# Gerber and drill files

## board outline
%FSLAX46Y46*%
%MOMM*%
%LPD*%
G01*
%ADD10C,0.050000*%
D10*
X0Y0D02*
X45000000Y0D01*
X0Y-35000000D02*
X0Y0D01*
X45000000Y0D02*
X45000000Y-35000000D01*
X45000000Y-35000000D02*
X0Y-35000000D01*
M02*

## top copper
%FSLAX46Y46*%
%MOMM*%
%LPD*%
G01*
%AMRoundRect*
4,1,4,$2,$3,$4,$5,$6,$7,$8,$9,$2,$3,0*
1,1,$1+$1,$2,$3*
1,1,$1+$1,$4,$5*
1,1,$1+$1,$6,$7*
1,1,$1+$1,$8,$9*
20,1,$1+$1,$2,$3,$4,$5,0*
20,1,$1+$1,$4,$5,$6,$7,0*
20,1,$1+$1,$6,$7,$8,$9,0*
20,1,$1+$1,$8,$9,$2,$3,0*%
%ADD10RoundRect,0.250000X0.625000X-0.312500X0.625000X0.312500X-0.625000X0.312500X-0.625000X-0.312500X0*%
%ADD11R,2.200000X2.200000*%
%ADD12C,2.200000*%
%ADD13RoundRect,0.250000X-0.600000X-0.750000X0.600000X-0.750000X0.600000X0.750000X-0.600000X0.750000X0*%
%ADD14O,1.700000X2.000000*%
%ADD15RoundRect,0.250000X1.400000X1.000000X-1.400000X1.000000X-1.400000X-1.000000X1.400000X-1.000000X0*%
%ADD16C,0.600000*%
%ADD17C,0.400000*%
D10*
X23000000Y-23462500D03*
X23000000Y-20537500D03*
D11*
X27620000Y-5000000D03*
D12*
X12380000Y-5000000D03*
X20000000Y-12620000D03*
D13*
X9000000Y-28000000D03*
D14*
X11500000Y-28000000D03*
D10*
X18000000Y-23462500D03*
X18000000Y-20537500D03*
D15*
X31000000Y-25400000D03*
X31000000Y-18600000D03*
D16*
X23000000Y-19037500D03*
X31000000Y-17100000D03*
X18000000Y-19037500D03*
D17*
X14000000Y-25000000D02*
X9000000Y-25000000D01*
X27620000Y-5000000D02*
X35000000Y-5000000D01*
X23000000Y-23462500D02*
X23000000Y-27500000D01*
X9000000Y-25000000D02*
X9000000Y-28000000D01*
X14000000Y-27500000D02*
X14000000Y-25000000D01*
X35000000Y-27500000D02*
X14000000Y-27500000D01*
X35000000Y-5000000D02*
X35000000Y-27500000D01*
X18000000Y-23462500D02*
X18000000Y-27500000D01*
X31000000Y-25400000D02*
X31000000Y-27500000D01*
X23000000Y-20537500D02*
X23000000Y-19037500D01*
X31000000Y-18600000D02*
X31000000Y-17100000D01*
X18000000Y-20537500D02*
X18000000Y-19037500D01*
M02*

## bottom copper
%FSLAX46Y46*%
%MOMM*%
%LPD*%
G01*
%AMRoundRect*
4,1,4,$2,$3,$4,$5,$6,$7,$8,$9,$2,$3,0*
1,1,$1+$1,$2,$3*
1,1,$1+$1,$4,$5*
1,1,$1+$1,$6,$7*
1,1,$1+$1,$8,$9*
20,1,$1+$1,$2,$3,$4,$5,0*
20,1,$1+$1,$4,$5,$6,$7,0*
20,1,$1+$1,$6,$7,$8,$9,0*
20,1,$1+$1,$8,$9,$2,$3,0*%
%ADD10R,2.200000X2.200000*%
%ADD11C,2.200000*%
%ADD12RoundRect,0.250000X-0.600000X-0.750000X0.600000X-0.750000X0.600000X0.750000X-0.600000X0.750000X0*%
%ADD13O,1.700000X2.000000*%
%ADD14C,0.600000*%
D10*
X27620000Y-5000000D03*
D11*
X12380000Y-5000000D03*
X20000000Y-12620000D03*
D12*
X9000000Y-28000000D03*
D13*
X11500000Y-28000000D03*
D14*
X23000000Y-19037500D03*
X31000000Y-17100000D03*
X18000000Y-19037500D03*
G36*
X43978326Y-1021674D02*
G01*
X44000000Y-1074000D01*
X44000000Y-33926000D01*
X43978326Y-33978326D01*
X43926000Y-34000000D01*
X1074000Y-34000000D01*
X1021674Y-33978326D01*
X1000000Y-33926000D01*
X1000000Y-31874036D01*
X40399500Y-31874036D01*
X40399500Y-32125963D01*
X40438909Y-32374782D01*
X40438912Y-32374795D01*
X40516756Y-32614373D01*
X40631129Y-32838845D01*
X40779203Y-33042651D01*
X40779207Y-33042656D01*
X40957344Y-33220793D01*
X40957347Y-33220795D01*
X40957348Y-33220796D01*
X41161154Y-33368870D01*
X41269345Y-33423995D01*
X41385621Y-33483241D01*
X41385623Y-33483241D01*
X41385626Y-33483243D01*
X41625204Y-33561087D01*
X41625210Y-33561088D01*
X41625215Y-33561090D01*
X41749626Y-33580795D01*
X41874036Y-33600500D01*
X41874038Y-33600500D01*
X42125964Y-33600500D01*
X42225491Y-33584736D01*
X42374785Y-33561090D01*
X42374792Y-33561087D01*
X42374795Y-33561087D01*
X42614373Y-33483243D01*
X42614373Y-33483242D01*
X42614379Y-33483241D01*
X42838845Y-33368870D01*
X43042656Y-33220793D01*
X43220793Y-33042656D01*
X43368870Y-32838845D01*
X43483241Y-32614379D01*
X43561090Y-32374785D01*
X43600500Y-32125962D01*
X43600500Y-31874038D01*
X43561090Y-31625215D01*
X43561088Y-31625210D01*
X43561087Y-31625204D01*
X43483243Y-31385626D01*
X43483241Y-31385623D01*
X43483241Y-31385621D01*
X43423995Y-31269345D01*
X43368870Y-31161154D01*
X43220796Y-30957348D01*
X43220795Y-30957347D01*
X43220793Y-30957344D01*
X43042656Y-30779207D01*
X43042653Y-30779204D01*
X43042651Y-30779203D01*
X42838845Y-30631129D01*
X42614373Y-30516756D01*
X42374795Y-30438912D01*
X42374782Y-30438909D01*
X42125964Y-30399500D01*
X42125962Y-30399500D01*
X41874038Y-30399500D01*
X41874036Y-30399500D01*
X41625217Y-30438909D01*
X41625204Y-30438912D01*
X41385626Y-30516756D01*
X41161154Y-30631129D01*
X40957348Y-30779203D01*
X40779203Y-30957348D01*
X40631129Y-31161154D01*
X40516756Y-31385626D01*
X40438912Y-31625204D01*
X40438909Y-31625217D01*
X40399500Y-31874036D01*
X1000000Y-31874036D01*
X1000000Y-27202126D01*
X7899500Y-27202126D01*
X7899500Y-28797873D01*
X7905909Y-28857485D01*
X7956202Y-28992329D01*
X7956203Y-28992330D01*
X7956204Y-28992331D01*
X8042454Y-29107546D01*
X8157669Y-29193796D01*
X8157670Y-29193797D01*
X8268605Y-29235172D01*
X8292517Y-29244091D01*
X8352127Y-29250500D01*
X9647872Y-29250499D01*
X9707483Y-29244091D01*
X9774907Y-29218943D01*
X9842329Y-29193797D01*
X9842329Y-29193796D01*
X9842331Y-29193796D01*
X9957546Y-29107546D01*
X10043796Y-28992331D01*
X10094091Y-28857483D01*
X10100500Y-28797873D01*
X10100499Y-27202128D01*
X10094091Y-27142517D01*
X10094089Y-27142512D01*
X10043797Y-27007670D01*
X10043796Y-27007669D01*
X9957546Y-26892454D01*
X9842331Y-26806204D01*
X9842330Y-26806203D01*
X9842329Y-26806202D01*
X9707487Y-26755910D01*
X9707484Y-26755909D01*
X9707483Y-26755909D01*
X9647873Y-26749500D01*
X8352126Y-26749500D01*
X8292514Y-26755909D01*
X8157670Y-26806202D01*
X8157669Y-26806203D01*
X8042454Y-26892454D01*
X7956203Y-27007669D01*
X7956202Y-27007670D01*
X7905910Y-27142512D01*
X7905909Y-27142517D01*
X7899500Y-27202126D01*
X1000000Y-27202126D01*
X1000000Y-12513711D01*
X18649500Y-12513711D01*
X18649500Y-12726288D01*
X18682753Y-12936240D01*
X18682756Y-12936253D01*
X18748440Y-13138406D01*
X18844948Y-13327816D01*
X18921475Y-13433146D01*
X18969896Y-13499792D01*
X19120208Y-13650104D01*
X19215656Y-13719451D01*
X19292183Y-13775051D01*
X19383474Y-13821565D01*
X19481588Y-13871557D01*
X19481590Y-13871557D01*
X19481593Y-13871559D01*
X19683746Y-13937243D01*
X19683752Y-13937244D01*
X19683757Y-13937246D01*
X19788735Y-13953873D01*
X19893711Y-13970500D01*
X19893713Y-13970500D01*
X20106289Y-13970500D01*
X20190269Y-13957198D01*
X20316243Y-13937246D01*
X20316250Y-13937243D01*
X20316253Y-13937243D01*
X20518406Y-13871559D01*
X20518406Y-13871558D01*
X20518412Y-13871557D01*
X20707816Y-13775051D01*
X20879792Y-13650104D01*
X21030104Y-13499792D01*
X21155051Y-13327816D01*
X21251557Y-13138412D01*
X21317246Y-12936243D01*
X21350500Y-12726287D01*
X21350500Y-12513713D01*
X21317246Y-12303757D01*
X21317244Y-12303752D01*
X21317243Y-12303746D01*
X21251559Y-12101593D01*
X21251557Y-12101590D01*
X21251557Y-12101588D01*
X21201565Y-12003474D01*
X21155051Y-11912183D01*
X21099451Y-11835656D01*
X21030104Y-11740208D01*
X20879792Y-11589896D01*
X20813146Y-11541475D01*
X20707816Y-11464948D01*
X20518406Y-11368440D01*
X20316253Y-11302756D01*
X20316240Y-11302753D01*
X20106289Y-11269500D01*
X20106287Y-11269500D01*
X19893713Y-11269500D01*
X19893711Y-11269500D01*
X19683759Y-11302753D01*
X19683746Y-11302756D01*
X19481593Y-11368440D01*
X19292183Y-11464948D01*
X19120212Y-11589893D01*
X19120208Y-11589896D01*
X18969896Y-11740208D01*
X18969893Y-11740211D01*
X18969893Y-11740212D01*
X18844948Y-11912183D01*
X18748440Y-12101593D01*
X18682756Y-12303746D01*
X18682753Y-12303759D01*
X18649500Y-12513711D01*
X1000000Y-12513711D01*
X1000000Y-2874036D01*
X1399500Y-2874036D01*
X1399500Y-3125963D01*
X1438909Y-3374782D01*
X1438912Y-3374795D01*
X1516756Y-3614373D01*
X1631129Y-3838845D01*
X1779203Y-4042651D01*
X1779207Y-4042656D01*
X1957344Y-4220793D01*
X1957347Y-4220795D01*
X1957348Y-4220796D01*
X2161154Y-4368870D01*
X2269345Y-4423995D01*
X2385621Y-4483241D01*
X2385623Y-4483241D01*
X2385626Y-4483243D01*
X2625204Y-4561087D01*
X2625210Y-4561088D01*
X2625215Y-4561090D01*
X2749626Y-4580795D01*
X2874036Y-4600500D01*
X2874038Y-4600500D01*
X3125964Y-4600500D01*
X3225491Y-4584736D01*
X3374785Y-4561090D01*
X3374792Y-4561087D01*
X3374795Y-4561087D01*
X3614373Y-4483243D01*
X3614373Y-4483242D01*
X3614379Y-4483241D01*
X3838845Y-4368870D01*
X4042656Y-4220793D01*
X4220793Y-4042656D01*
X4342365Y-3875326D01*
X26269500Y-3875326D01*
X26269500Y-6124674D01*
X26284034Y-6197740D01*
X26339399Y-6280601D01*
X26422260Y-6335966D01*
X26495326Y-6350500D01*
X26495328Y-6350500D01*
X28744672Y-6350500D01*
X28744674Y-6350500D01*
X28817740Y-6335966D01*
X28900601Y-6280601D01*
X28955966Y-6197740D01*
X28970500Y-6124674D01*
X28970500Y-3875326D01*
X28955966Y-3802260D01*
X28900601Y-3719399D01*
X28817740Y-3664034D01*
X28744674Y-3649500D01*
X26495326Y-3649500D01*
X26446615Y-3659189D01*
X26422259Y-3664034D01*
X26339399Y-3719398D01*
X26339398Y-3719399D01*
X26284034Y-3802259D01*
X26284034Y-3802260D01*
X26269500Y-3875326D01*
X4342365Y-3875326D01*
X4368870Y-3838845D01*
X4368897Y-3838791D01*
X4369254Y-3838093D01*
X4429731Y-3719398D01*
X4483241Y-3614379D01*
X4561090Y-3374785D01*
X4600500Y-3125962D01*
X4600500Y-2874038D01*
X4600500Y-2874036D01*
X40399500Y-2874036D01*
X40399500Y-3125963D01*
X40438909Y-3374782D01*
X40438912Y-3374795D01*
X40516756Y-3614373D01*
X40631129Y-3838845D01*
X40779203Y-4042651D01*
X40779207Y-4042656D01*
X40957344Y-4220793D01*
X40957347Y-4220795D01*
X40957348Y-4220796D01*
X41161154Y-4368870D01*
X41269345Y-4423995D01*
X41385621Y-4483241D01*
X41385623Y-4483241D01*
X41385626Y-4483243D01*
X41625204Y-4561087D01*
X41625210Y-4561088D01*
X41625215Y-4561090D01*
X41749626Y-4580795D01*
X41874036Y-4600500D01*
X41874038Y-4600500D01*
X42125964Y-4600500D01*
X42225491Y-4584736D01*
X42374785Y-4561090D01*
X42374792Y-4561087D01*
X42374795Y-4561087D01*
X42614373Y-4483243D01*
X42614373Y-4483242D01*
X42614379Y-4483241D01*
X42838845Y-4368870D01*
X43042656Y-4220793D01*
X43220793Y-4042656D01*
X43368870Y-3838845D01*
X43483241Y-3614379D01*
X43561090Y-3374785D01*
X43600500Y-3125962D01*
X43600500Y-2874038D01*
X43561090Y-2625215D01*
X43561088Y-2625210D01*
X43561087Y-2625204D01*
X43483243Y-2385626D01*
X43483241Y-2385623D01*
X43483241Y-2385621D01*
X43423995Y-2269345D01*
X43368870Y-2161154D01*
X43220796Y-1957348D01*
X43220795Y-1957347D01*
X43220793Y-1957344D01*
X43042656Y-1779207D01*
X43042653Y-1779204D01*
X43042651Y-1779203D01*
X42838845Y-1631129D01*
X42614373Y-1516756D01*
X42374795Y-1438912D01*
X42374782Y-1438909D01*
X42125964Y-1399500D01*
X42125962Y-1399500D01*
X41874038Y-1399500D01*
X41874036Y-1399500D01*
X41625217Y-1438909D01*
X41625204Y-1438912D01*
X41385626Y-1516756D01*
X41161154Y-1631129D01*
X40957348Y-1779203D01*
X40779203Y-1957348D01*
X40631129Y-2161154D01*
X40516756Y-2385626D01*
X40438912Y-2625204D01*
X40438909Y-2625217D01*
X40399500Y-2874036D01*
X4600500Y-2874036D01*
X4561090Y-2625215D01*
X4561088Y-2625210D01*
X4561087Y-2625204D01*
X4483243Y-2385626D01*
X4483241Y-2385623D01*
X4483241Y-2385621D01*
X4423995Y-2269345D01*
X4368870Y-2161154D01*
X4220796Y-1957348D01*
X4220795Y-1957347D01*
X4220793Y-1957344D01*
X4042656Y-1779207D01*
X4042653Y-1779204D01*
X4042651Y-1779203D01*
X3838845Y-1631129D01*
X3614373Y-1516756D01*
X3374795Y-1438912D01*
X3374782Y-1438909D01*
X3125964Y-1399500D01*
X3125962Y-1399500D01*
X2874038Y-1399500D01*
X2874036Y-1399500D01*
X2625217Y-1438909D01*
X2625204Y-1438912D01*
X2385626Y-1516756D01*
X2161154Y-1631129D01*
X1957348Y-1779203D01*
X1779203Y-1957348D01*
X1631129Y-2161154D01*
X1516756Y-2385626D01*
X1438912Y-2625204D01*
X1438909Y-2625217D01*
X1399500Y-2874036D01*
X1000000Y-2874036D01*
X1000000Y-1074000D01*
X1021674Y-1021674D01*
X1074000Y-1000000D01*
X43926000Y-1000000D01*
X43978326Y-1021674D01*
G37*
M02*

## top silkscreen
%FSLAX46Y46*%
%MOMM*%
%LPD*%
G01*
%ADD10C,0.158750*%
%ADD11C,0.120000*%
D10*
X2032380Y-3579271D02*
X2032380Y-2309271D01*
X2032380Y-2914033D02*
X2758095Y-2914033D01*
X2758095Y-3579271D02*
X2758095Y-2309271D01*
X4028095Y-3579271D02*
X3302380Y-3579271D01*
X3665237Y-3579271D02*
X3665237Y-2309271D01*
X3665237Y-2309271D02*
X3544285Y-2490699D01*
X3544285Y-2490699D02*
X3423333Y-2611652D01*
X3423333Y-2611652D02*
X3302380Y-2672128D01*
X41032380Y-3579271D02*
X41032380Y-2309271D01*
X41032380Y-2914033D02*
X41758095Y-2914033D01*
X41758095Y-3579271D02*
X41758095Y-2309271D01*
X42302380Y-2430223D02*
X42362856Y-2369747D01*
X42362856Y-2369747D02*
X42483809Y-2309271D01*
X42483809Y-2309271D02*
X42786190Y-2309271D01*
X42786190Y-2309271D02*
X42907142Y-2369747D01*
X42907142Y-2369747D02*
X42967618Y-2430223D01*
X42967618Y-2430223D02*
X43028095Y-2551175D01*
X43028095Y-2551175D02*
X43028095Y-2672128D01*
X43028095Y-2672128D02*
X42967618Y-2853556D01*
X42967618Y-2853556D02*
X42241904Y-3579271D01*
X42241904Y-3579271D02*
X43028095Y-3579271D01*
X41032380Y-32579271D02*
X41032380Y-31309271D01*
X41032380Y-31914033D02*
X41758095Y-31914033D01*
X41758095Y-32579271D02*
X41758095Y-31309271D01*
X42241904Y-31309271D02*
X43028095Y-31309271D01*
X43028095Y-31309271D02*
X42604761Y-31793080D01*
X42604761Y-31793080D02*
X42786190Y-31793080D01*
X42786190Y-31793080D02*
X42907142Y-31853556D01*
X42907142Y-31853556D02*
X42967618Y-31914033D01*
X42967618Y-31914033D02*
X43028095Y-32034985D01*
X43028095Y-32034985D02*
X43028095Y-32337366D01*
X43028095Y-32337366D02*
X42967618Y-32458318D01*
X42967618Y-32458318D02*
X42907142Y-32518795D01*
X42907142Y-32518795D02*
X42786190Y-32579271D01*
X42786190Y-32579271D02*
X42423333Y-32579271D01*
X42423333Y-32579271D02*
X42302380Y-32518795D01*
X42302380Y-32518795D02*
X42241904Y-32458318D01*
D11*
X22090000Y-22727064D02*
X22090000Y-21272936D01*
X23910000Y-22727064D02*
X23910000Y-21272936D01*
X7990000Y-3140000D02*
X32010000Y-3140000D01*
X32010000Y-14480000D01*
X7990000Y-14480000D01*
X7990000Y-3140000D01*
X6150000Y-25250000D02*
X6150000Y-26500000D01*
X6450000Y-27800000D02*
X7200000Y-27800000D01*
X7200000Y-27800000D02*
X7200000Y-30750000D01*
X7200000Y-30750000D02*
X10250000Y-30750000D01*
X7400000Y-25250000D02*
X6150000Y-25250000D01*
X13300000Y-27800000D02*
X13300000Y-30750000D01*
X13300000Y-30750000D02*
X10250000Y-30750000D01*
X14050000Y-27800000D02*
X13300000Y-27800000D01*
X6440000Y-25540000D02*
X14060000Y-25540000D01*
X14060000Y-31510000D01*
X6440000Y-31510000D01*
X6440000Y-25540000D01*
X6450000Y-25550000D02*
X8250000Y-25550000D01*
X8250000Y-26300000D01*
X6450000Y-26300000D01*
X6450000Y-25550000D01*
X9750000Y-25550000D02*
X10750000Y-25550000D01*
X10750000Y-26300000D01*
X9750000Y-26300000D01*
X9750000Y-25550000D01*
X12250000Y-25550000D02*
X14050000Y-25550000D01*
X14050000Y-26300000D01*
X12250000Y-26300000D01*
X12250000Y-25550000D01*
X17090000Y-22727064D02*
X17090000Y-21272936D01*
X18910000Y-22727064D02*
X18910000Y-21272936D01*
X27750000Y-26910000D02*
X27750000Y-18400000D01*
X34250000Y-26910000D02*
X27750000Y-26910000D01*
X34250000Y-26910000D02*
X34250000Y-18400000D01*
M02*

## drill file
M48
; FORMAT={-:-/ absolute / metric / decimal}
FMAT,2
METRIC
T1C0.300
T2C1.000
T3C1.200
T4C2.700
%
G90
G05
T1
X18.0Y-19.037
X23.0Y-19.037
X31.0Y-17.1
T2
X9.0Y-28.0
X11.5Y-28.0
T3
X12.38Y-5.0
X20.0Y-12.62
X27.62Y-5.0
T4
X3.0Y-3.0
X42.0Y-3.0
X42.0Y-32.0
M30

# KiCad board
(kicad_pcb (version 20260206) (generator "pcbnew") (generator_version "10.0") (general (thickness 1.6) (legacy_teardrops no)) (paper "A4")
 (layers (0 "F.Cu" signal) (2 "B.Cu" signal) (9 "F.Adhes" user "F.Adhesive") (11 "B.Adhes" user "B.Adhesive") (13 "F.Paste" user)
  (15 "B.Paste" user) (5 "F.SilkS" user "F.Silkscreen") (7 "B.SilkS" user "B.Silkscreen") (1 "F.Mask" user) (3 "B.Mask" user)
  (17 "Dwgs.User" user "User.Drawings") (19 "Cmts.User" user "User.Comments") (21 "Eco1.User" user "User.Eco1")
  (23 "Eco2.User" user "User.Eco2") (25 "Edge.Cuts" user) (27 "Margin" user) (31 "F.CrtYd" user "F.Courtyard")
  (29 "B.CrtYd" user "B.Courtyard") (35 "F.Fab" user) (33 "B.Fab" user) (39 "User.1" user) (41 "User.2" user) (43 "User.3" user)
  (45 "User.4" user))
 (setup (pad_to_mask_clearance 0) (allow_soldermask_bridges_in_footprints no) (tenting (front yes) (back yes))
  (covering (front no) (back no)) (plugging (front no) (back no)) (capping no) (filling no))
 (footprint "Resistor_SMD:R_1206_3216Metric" (layer "F.Cu") (at 23 22 90)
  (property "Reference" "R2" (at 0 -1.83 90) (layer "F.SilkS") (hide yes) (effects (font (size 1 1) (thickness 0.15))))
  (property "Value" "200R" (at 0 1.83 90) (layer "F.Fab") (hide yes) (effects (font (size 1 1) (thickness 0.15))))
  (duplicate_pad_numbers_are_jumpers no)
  (fp_line (start -0.727064 -0.91) (end 0.727064 -0.91) (stroke (width 0.12) (type solid)) (layer "F.SilkS"))
  (fp_line (start -0.727064 0.91) (end 0.727064 0.91) (stroke (width 0.12) (type solid)) (layer "F.SilkS"))
  (pad "1" smd roundrect (at -1.4625 0 90) (size 1.125 1.75) (layers "F.Cu" "F.Mask" "F.Paste") (roundrect_rratio 0.222222)
   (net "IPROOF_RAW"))
  (pad "2" smd roundrect (at 1.4625 0 90) (size 1.125 1.75) (layers "F.Cu" "F.Mask" "F.Paste") (roundrect_rratio 0.222222) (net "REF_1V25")))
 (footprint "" (layer "F.Cu") (at 3 3)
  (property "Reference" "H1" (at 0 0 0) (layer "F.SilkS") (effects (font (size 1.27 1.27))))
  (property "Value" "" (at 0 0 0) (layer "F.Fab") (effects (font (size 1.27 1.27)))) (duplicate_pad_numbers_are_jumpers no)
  (pad "" np_thru_hole circle (at 0 0) (size 2.7 2.7) (drill 2.7) (layers "*.Cu")))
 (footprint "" (layer "F.Cu") (at 42 3)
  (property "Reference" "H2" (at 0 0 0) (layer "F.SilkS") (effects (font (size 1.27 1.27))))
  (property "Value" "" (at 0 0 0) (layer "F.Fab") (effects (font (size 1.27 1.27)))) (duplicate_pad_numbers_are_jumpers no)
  (pad "" np_thru_hole circle (at 0 0) (size 2.7 2.7) (drill 2.7) (layers "*.Cu")))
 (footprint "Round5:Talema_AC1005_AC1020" (layer "F.Cu") (at 20 5)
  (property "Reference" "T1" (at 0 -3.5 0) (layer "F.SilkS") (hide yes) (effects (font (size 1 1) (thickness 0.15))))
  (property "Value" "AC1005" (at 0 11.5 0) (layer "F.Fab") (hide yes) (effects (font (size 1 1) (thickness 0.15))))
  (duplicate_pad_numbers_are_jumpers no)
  (fp_rect (start -12.01 -1.86) (end 12.01 9.48) (stroke (width 0.12) (type default)) (fill no) (layer "F.SilkS"))
  (pad "1" thru_hole rect (at 7.62 0) (size 2.2 2.2) (drill 1.2) (layers "*.Cu" "*.Mask") (remove_unused_layers no) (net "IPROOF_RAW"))
  (pad "2" thru_hole circle (at -7.62 0) (size 2.2 2.2) (drill 1.2) (layers "*.Cu" "*.Mask") (remove_unused_layers no) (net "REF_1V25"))
  (pad "3" thru_hole circle (at 0 7.62) (size 2.2 2.2) (drill 1.2) (layers "*.Cu" "*.Mask") (remove_unused_layers no)
   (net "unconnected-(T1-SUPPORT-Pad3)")))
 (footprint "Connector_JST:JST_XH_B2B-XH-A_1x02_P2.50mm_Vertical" (layer "F.Cu") (at 9 28)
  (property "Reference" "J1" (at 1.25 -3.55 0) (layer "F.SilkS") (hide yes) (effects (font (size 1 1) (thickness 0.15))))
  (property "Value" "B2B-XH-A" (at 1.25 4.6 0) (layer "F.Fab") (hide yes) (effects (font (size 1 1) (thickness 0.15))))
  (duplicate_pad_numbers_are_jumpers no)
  (fp_line (start -2.85 -2.75) (end -2.85 -1.5) (stroke (width 0.12) (type solid)) (layer "F.SilkS"))
  (fp_line (start -2.55 -0.2) (end -1.8 -0.2) (stroke (width 0.12) (type solid)) (layer "F.SilkS"))
  (fp_line (start -1.8 -0.2) (end -1.8 2.75) (stroke (width 0.12) (type solid)) (layer "F.SilkS"))
  (fp_line (start -1.8 2.75) (end 1.25 2.75) (stroke (width 0.12) (type solid)) (layer "F.SilkS"))
  (fp_line (start -1.6 -2.75) (end -2.85 -2.75) (stroke (width 0.12) (type solid)) (layer "F.SilkS"))
  (fp_line (start 4.3 -0.2) (end 4.3 2.75) (stroke (width 0.12) (type solid)) (layer "F.SilkS"))
  (fp_line (start 4.3 2.75) (end 1.25 2.75) (stroke (width 0.12) (type solid)) (layer "F.SilkS"))
  (fp_line (start 5.05 -0.2) (end 4.3 -0.2) (stroke (width 0.12) (type solid)) (layer "F.SilkS"))
  (fp_rect (start -2.56 -2.46) (end 5.06 3.51) (stroke (width 0.12) (type solid)) (fill no) (layer "F.SilkS"))
  (fp_rect (start -2.55 -2.45) (end -0.75 -1.7) (stroke (width 0.12) (type solid)) (fill no) (layer "F.SilkS"))
  (fp_rect (start 0.75 -2.45) (end 1.75 -1.7) (stroke (width 0.12) (type solid)) (fill no) (layer "F.SilkS"))
  (fp_rect (start 3.25 -2.45) (end 5.05 -1.7) (stroke (width 0.12) (type solid)) (fill no) (layer "F.SilkS"))
  (pad "1" thru_hole roundrect (at 0 0) (size 1.7 2) (drill 1) (layers "*.Cu" "*.Mask") (remove_unused_layers no)
   (roundrect_rratio 0.147059) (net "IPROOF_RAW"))
  (pad "2" thru_hole oval (at 2.5 0) (size 1.7 2) (drill 1) (layers "*.Cu" "*.Mask") (remove_unused_layers no) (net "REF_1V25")))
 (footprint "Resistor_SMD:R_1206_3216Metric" (layer "F.Cu") (at 18 22 90)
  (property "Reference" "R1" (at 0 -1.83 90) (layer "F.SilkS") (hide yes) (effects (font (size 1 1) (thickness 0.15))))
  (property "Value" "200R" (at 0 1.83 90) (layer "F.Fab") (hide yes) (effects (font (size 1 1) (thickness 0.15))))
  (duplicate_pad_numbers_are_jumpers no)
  (fp_line (start -0.727064 -0.91) (end 0.727064 -0.91) (stroke (width 0.12) (type solid)) (layer "F.SilkS"))
  (fp_line (start -0.727064 0.91) (end 0.727064 0.91) (stroke (width 0.12) (type solid)) (layer "F.SilkS"))
  (pad "1" smd roundrect (at -1.4625 0 90) (size 1.125 1.75) (layers "F.Cu" "F.Mask" "F.Paste") (roundrect_rratio 0.222222)
   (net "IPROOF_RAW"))
  (pad "2" smd roundrect (at 1.4625 0 90) (size 1.125 1.75) (layers "F.Cu" "F.Mask" "F.Paste") (roundrect_rratio 0.222222) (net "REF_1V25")))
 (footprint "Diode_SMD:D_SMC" (layer "F.Cu") (at 31 22 90)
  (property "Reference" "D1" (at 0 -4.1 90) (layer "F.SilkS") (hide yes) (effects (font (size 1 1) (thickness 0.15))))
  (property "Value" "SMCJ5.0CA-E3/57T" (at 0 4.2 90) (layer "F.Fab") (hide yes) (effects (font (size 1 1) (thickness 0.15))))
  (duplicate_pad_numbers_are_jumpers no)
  (fp_line (start -4.91 -3.25) (end 3.6 -3.25) (stroke (width 0.12) (type solid)) (layer "F.SilkS"))
  (fp_line (start -4.91 3.25) (end -4.91 -3.25) (stroke (width 0.12) (type solid)) (layer "F.SilkS"))
  (fp_line (start -4.91 3.25) (end 3.6 3.25) (stroke (width 0.12) (type solid)) (layer "F.SilkS"))
  (pad "1" smd roundrect (at -3.4 0 180) (size 3.3 2.5) (layers "F.Cu" "F.Mask" "F.Paste") (roundrect_rratio 0.1) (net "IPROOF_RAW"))
  (pad "2" smd roundrect (at 3.4 0 180) (size 3.3 2.5) (layers "F.Cu" "F.Mask" "F.Paste") (roundrect_rratio 0.1) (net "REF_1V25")))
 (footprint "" (layer "F.Cu") (at 42 32)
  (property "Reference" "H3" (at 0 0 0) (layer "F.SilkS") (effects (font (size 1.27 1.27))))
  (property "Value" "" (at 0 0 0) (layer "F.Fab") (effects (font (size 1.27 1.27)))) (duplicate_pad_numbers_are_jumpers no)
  (pad "" np_thru_hole circle (at 0 0) (size 2.7 2.7) (drill 2.7) (layers "*.Cu")))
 (gr_line (start 0 0) (end 45 0) (stroke (width 0.05) (type default)) (layer "Edge.Cuts"))
 (gr_line (start 0 35) (end 0 0) (stroke (width 0.05) (type default)) (layer "Edge.Cuts"))
 (gr_line (start 45 0) (end 45 35) (stroke (width 0.05) (type default)) (layer "Edge.Cuts"))
 (gr_line (start 45 35) (end 0 35) (stroke (width 0.05) (type default)) (layer "Edge.Cuts"))
 (segment (start 14 25) (end 9 25) (width 0.4) (layer "F.Cu") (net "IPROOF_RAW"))
 (segment (start 27.62 5) (end 35 5) (width 0.4) (layer "F.Cu") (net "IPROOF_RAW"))
 (segment (start 23 23.4625) (end 23 27.5) (width 0.4) (layer "F.Cu") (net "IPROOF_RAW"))
 (segment (start 9 25) (end 9 28) (width 0.4) (layer "F.Cu") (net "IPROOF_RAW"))
 (segment (start 14 27.5) (end 14 25) (width 0.4) (layer "F.Cu") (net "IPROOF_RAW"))
 (segment (start 35 27.5) (end 14 27.5) (width 0.4) (layer "F.Cu") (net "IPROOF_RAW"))
 (segment (start 35 5) (end 35 27.5) (width 0.4) (layer "F.Cu") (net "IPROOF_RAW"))
 (segment (start 18 23.4625) (end 18 27.5) (width 0.4) (layer "F.Cu") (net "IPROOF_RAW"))
 (segment (start 31 25.4) (end 31 27.5) (width 0.4) (layer "F.Cu") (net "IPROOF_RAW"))
 (segment (start 23 20.5375) (end 23 19.0375) (width 0.4) (layer "F.Cu") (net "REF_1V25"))
 (segment (start 31 18.6) (end 31 17.1) (width 0.4) (layer "F.Cu") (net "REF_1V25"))
 (segment (start 18 20.5375) (end 18 19.0375) (width 0.4) (layer "F.Cu") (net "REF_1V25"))
 (via (at 23 19.0375) (size 0.6) (drill 0.3) (layers "F.Cu" "B.Cu") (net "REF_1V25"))
 (via (at 31 17.1) (size 0.6) (drill 0.3) (layers "F.Cu" "B.Cu") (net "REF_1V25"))
 (via (at 18 19.0375) (size 0.6) (drill 0.3) (layers "F.Cu" "B.Cu") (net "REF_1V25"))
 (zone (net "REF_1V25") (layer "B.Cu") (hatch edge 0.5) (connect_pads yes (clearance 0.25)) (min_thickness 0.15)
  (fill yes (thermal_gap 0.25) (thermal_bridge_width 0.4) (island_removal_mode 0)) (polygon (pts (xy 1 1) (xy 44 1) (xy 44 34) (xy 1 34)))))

